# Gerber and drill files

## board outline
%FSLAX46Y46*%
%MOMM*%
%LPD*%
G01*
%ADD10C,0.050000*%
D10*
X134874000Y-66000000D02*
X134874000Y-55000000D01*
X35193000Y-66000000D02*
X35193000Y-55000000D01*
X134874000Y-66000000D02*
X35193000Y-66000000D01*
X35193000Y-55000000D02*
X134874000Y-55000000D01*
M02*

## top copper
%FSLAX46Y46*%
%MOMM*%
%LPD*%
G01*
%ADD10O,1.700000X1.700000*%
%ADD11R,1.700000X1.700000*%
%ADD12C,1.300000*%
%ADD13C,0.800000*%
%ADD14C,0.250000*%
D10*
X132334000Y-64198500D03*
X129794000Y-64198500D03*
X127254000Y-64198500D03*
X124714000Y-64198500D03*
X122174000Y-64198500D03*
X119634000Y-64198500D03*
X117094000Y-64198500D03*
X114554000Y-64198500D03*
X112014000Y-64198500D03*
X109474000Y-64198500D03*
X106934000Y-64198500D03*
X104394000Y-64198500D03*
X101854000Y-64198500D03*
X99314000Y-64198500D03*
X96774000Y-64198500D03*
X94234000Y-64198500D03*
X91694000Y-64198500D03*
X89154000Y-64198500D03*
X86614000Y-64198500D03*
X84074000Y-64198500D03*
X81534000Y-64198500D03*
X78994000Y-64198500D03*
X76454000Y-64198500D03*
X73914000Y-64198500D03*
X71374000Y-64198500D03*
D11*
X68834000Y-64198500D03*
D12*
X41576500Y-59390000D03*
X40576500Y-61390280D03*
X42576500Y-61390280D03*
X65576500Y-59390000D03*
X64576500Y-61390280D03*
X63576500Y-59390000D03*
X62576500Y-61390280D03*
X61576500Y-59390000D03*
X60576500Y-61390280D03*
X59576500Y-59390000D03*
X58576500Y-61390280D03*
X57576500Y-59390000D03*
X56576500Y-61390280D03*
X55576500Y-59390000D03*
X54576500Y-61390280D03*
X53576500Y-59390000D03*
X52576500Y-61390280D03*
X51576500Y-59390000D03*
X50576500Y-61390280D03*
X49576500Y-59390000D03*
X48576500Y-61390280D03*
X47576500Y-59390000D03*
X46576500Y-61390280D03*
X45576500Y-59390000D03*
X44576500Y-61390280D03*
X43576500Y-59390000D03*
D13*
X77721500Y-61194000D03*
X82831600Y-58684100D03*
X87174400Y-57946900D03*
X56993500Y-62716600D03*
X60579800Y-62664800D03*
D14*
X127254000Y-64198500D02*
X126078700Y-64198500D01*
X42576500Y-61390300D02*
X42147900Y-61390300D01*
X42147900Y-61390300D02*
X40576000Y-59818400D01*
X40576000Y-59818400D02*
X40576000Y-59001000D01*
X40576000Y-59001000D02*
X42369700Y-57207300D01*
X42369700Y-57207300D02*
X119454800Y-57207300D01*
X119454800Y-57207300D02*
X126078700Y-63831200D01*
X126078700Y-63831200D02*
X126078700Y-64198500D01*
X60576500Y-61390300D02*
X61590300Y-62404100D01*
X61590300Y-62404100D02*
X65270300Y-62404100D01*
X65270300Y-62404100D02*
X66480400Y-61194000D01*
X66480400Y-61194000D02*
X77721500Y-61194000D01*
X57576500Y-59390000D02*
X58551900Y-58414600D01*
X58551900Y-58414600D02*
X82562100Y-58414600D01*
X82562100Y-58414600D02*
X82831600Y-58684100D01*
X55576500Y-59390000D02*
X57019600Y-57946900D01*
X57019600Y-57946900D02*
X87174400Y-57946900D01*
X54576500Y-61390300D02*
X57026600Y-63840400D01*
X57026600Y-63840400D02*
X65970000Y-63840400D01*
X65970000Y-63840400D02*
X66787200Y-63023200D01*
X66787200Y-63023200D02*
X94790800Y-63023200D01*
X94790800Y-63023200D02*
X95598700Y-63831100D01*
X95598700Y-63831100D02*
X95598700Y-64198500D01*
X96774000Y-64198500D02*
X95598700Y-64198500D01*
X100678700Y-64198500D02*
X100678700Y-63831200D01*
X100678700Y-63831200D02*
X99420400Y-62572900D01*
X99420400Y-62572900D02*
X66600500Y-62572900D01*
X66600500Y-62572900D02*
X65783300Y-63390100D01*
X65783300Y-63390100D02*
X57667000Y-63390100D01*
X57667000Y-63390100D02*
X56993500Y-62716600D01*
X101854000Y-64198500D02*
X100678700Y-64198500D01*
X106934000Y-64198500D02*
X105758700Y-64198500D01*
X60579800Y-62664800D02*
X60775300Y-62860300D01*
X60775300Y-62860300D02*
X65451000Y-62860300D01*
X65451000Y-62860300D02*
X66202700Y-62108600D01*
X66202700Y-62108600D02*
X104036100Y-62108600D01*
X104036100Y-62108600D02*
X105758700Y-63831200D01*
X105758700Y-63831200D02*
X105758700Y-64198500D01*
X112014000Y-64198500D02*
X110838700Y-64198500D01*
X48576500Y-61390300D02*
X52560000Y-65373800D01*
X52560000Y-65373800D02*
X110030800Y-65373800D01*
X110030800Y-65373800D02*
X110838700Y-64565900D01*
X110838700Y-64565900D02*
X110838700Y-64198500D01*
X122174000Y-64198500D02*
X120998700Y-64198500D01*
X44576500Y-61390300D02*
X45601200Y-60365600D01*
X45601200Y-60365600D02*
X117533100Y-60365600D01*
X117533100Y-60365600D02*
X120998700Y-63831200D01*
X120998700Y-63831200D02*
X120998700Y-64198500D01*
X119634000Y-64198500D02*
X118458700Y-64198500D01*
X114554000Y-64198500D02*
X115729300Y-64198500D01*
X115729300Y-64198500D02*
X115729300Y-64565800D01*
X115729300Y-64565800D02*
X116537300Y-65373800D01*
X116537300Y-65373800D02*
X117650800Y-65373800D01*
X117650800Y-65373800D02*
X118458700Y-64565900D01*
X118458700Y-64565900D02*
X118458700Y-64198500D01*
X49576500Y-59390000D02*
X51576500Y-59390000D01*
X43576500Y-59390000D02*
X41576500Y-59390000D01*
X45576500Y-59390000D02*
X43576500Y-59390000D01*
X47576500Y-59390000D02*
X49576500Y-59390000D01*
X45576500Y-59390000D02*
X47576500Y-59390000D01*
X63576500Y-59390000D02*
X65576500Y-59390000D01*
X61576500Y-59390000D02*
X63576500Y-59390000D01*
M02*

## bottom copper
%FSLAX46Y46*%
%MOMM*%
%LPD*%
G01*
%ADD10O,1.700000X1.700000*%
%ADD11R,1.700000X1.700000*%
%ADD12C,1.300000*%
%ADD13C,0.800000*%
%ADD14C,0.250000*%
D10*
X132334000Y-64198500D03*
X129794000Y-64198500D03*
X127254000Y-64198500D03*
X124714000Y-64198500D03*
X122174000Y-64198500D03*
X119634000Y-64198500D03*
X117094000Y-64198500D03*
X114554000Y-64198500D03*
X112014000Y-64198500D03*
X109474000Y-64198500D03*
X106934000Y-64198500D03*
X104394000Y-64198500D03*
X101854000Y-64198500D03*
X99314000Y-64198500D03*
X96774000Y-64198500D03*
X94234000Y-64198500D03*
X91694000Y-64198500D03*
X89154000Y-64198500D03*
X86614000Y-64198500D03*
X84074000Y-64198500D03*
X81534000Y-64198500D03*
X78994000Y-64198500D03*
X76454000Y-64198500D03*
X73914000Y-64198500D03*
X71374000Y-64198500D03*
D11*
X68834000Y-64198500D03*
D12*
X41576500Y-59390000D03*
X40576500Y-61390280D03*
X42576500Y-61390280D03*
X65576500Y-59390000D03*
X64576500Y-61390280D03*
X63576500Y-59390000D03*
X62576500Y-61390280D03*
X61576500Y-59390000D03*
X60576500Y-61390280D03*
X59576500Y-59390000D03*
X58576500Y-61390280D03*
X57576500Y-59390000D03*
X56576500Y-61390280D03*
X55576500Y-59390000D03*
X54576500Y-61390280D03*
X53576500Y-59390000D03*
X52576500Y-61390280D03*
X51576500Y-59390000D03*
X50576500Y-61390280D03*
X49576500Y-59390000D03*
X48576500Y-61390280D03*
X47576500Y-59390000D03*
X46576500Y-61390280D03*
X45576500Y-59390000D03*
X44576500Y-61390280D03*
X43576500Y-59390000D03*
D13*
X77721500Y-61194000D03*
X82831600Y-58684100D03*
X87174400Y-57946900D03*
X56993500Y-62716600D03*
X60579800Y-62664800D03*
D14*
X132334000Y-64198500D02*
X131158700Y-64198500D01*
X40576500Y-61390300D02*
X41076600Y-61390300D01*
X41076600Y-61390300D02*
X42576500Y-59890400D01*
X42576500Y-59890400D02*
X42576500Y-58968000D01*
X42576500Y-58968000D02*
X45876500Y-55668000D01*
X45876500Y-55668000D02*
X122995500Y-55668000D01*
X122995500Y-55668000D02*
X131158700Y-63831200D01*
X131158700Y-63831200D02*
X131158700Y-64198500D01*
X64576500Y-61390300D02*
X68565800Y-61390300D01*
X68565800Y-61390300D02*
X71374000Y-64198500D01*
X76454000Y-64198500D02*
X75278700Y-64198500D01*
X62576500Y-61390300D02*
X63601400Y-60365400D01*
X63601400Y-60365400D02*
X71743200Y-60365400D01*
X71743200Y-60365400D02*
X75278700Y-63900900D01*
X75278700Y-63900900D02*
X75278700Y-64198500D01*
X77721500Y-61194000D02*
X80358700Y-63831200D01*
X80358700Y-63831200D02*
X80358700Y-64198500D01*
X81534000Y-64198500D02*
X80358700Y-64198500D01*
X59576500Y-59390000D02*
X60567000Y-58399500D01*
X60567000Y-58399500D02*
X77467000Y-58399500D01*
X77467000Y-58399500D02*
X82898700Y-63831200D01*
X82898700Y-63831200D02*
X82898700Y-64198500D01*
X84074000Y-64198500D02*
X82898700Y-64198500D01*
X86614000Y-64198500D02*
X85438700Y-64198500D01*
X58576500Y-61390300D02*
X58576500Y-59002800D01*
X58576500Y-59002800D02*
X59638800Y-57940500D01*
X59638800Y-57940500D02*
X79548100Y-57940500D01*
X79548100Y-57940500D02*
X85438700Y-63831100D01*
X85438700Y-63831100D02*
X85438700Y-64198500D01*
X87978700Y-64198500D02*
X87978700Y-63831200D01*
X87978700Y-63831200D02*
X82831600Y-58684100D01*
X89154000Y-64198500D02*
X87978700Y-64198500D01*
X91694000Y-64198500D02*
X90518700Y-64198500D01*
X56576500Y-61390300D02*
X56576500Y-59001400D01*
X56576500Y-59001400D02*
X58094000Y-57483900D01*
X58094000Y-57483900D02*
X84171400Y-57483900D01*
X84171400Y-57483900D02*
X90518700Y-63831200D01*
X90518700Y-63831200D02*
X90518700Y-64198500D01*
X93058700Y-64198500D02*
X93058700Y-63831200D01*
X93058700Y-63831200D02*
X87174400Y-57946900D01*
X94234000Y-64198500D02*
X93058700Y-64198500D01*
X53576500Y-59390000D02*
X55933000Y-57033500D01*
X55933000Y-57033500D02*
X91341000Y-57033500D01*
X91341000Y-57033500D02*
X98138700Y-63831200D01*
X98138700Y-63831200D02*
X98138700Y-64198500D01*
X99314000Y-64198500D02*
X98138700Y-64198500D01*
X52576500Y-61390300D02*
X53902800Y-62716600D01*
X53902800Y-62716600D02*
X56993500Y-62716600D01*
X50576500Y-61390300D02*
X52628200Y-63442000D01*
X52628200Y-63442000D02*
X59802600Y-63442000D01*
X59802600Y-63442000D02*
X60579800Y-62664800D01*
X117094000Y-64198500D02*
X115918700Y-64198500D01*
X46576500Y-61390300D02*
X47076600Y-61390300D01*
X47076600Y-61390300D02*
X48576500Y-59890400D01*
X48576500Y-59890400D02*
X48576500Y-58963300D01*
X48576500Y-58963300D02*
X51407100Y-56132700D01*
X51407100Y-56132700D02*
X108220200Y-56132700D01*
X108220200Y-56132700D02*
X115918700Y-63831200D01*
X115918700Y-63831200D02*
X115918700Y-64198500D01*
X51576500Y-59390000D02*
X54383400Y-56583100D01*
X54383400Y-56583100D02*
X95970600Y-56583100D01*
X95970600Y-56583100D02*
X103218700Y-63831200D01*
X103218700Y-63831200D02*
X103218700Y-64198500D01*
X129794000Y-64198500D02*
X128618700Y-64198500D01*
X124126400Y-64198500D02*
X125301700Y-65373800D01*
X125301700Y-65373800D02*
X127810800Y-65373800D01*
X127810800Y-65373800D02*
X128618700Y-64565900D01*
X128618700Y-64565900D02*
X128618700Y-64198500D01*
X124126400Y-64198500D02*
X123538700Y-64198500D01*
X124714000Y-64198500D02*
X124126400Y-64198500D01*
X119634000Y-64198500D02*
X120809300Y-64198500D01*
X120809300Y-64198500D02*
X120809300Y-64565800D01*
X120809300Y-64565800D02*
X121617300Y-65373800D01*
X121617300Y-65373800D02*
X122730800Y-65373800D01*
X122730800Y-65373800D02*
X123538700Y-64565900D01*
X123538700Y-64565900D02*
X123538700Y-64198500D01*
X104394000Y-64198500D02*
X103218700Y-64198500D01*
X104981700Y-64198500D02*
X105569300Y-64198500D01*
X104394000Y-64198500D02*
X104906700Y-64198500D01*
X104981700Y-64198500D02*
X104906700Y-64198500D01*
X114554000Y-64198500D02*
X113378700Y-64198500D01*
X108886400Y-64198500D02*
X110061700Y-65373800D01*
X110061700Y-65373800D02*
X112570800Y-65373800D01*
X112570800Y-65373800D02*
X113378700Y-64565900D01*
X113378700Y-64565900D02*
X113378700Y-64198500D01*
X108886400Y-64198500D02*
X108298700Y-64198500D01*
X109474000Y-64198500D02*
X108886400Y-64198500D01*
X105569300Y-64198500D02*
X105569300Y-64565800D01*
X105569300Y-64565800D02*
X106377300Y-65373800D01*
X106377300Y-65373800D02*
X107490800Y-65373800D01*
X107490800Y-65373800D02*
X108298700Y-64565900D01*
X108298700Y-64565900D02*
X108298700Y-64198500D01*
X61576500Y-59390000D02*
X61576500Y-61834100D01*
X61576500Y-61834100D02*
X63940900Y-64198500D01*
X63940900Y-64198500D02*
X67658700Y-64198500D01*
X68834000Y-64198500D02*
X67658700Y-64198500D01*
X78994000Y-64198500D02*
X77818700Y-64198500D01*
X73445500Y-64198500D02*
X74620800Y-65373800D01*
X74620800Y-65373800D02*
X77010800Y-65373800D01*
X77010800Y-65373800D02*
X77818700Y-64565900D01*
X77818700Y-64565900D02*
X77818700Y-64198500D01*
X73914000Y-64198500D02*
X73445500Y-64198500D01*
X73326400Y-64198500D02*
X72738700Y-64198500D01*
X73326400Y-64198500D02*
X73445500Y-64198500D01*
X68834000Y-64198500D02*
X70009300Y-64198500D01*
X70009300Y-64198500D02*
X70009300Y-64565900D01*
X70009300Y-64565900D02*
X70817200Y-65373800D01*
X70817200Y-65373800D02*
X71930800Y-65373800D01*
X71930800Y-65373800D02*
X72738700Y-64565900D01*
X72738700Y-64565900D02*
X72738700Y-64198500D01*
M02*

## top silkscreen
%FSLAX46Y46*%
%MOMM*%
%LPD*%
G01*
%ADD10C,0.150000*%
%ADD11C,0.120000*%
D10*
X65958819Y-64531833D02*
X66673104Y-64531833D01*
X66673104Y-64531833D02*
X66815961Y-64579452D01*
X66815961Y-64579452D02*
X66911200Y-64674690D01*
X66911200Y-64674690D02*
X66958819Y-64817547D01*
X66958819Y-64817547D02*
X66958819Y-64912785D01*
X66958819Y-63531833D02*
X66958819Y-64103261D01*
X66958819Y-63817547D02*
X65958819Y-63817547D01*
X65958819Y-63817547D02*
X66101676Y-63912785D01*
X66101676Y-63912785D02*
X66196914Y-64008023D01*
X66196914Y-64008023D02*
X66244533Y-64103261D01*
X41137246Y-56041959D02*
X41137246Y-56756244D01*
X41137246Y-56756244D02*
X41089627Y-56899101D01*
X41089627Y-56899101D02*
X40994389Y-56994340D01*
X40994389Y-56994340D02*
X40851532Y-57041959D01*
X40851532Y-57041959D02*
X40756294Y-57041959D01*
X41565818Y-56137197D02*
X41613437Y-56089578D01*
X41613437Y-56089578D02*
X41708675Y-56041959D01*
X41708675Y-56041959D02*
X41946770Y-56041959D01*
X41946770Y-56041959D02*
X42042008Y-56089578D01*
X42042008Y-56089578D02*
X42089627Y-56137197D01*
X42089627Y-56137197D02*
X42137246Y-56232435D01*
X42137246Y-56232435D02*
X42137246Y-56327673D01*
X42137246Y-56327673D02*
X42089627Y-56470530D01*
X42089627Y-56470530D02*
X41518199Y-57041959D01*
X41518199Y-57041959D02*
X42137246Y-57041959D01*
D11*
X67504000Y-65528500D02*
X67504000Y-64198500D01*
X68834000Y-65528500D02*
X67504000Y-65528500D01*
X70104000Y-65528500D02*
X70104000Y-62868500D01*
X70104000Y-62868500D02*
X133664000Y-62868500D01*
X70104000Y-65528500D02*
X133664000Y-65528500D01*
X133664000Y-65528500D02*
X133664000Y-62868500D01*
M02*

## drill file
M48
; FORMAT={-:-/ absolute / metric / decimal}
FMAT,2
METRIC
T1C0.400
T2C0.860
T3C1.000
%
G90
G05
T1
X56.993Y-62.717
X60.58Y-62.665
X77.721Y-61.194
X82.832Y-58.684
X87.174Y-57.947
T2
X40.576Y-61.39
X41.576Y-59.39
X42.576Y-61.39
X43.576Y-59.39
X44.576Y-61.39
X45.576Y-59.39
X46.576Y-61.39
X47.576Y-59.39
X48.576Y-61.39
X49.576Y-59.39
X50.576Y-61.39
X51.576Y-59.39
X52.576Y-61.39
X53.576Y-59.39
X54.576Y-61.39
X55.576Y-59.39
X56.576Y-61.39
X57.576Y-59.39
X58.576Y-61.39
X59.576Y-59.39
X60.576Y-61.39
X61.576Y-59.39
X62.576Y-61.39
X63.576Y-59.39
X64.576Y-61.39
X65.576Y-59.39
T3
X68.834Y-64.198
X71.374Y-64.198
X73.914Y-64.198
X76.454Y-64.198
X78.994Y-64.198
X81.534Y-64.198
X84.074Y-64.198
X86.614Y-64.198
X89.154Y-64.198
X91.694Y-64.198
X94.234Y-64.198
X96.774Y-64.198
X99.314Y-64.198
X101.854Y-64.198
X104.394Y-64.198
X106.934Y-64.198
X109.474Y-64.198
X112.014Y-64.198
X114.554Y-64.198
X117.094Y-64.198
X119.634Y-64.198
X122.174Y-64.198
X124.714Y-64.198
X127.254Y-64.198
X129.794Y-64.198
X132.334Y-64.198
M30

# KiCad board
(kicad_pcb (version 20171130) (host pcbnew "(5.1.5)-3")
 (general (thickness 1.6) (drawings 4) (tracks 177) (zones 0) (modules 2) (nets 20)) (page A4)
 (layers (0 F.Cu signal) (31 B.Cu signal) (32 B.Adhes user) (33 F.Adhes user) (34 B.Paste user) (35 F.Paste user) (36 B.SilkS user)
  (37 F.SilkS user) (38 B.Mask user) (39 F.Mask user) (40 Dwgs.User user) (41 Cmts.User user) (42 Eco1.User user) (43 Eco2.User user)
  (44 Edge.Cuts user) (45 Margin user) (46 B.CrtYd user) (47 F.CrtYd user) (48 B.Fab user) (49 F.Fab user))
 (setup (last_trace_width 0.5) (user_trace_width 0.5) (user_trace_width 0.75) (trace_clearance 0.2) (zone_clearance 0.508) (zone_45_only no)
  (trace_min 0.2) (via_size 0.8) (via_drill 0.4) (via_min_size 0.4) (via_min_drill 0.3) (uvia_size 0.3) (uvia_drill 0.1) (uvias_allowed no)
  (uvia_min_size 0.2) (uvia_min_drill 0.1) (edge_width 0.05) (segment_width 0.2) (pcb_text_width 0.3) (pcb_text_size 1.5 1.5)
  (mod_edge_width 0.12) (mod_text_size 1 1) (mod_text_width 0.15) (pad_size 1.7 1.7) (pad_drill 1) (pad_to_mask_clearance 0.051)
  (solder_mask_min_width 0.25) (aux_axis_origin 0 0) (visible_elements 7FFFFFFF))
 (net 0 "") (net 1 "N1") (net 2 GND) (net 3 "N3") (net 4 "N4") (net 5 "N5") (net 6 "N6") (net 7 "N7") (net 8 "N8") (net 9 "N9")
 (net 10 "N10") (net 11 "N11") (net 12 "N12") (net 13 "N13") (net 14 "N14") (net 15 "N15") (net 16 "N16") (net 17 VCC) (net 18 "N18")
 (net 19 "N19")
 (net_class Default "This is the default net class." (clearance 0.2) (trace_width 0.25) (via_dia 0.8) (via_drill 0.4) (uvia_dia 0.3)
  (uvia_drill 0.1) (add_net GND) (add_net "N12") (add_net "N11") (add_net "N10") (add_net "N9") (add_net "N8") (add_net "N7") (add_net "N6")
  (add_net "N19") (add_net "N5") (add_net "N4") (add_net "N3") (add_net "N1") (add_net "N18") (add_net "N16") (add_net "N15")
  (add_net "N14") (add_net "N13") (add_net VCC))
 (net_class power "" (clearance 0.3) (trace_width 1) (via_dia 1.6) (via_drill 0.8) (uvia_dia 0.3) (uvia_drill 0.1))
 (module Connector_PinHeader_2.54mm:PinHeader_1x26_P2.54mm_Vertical (layer F.Cu) (at 68.834 64.1985 90)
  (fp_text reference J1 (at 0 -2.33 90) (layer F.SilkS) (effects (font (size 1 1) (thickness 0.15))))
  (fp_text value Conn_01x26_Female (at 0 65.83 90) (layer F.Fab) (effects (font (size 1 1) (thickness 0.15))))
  (fp_line (start -1.33 -1.33) (end 0 -1.33) (layer F.SilkS) (width 0.12))
  (fp_line (start -1.33 0) (end -1.33 -1.33) (layer F.SilkS) (width 0.12))
  (fp_line (start -1.33 1.27) (end 1.33 1.27) (layer F.SilkS) (width 0.12))
  (fp_line (start 1.33 1.27) (end 1.33 64.83) (layer F.SilkS) (width 0.12))
  (fp_line (start -1.33 1.27) (end -1.33 64.83) (layer F.SilkS) (width 0.12))
  (fp_line (start -1.33 64.83) (end 1.33 64.83) (layer F.SilkS) (width 0.12))
  (pad 26 thru_hole oval (at 0 63.5 90) (size 1.7 1.7) (drill 1) (layers *.Cu *.Mask) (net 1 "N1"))
  (pad 25 thru_hole oval (at 0 60.96 90) (size 1.7 1.7) (drill 1) (layers *.Cu *.Mask) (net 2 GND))
  (pad 24 thru_hole oval (at 0 58.42 90) (size 1.7 1.7) (drill 1) (layers *.Cu *.Mask) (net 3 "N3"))
  (pad 23 thru_hole oval (at 0 55.88 90) (size 1.7 1.7) (drill 1) (layers *.Cu *.Mask) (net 2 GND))
  (pad 22 thru_hole oval (at 0 53.34 90) (size 1.7 1.7) (drill 1) (layers *.Cu *.Mask) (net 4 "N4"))
  (pad 21 thru_hole oval (at 0 50.8 90) (size 1.7 1.7) (drill 1) (layers *.Cu *.Mask) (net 2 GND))
  (pad 20 thru_hole oval (at 0 48.26 90) (size 1.7 1.7) (drill 1) (layers *.Cu *.Mask) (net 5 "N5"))
  (pad 19 thru_hole oval (at 0 45.72 90) (size 1.7 1.7) (drill 1) (layers *.Cu *.Mask) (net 2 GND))
  (pad 18 thru_hole oval (at 0 43.18 90) (size 1.7 1.7) (drill 1) (layers *.Cu *.Mask) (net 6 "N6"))
  (pad 17 thru_hole oval (at 0 40.64 90) (size 1.7 1.7) (drill 1) (layers *.Cu *.Mask) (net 2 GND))
  (pad 16 thru_hole oval (at 0 38.1 90) (size 1.7 1.7) (drill 1) (layers *.Cu *.Mask) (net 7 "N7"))
  (pad 15 thru_hole oval (at 0 35.56 90) (size 1.7 1.7) (drill 1) (layers *.Cu *.Mask) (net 2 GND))
  (pad 14 thru_hole oval (at 0 33.02 90) (size 1.7 1.7) (drill 1) (layers *.Cu *.Mask) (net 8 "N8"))
  (pad 13 thru_hole oval (at 0 30.48 90) (size 1.7 1.7) (drill 1) (layers *.Cu *.Mask) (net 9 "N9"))
  (pad 12 thru_hole oval (at 0 27.94 90) (size 1.7 1.7) (drill 1) (layers *.Cu *.Mask) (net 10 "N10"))
  (pad 11 thru_hole oval (at 0 25.4 90) (size 1.7 1.7) (drill 1) (layers *.Cu *.Mask) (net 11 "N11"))
  (pad 10 thru_hole oval (at 0 22.86 90) (size 1.7 1.7) (drill 1) (layers *.Cu *.Mask) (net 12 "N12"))
  (pad 9 thru_hole oval (at 0 20.32 90) (size 1.7 1.7) (drill 1) (layers *.Cu *.Mask) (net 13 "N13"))
  (pad 8 thru_hole oval (at 0 17.78 90) (size 1.7 1.7) (drill 1) (layers *.Cu *.Mask) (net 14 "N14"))
  (pad 7 thru_hole oval (at 0 15.24 90) (size 1.7 1.7) (drill 1) (layers *.Cu *.Mask) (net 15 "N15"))
  (pad 6 thru_hole oval (at 0 12.7 90) (size 1.7 1.7) (drill 1) (layers *.Cu *.Mask) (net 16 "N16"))
  (pad 5 thru_hole oval (at 0 10.16 90) (size 1.7 1.7) (drill 1) (layers *.Cu *.Mask) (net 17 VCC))
  (pad 4 thru_hole oval (at 0 7.62 90) (size 1.7 1.7) (drill 1) (layers *.Cu *.Mask) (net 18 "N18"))
  (pad 3 thru_hole oval (at 0 5.08 90) (size 1.7 1.7) (drill 1) (layers *.Cu *.Mask) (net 17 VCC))
  (pad 2 thru_hole oval (at 0 2.54 90) (size 1.7 1.7) (drill 1) (layers *.Cu *.Mask) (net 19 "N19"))
  (pad 1 thru_hole rect (at 0 0 90) (size 1.7 1.7) (drill 1) (layers *.Cu *.Mask) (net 17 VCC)))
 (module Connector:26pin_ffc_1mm (layer F.Cu) (at 40.5765 64.103)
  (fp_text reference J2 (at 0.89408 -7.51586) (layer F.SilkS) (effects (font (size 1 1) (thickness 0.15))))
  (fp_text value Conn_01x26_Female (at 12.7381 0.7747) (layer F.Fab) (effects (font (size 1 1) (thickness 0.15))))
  (pad 25 thru_hole circle (at 1 -4.713) (size 1.3 1.3) (drill 0.86) (layers *.Cu *.Mask) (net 2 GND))
  (pad 26 thru_hole circle (at 0 -2.71272) (size 1.3 1.3) (drill 0.86) (layers *.Cu *.Mask) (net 1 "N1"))
  (pad 24 thru_hole circle (at 2 -2.71272) (size 1.3 1.3) (drill 0.86) (layers *.Cu *.Mask) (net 3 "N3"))
  (pad 1 thru_hole circle (at 25 -4.713) (size 1.3 1.3) (drill 0.86) (layers *.Cu *.Mask) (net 17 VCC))
  (pad 2 thru_hole circle (at 24 -2.71272) (size 1.3 1.3) (drill 0.86) (layers *.Cu *.Mask) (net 19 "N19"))
  (pad 3 thru_hole circle (at 23 -4.713) (size 1.3 1.3) (drill 0.86) (layers *.Cu *.Mask) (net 17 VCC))
  (pad 4 thru_hole circle (at 22 -2.71272) (size 1.3 1.3) (drill 0.86) (layers *.Cu *.Mask) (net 18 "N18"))
  (pad 5 thru_hole circle (at 21 -4.713) (size 1.3 1.3) (drill 0.86) (layers *.Cu *.Mask) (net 17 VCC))
  (pad 6 thru_hole circle (at 20 -2.71272) (size 1.3 1.3) (drill 0.86) (layers *.Cu *.Mask) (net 16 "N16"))
  (pad 7 thru_hole circle (at 19 -4.713) (size 1.3 1.3) (drill 0.86) (layers *.Cu *.Mask) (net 15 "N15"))
  (pad 8 thru_hole circle (at 18 -2.71272) (size 1.3 1.3) (drill 0.86) (layers *.Cu *.Mask) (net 14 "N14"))
  (pad 9 thru_hole circle (at 17 -4.713) (size 1.3 1.3) (drill 0.86) (layers *.Cu *.Mask) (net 13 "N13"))
  (pad 10 thru_hole circle (at 16 -2.71272) (size 1.3 1.3) (drill 0.86) (layers *.Cu *.Mask) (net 12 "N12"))
  (pad 11 thru_hole circle (at 15 -4.713) (size 1.3 1.3) (drill 0.86) (layers *.Cu *.Mask) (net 11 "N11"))
  (pad 12 thru_hole circle (at 14 -2.71272) (size 1.3 1.3) (drill 0.86) (layers *.Cu *.Mask) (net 10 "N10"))
  (pad 13 thru_hole circle (at 13 -4.713) (size 1.3 1.3) (drill 0.86) (layers *.Cu *.Mask) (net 9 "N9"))
  (pad 14 thru_hole circle (at 12 -2.71272) (size 1.3 1.3) (drill 0.86) (layers *.Cu *.Mask) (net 8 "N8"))
  (pad 15 thru_hole circle (at 11 -4.713) (size 1.3 1.3) (drill 0.86) (layers *.Cu *.Mask) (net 2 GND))
  (pad 16 thru_hole circle (at 10 -2.71272) (size 1.3 1.3) (drill 0.86) (layers *.Cu *.Mask) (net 7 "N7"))
  (pad 17 thru_hole circle (at 9 -4.713) (size 1.3 1.3) (drill 0.86) (layers *.Cu *.Mask) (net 2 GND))
  (pad 18 thru_hole circle (at 8 -2.71272) (size 1.3 1.3) (drill 0.86) (layers *.Cu *.Mask) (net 6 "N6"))
  (pad 19 thru_hole circle (at 7 -4.713) (size 1.3 1.3) (drill 0.86) (layers *.Cu *.Mask) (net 2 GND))
  (pad 20 thru_hole circle (at 6 -2.71272) (size 1.3 1.3) (drill 0.86) (layers *.Cu *.Mask) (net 5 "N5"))
  (pad 21 thru_hole circle (at 5 -4.713) (size 1.3 1.3) (drill 0.86) (layers *.Cu *.Mask) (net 2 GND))
  (pad 22 thru_hole circle (at 4 -2.71272) (size 1.3 1.3) (drill 0.86) (layers *.Cu *.Mask) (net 4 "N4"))
  (pad 23 thru_hole circle (at 3 -4.713) (size 1.3 1.3) (drill 0.86) (layers *.Cu *.Mask) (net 2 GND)))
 (gr_line (start 134.874 66) (end 134.874 55) (layer Edge.Cuts) (width 0.05))
 (gr_line (start 35.193 66) (end 35.193 55) (layer Edge.Cuts) (width 0.05))
 (gr_line (start 134.874 66) (end 35.193 66) (layer Edge.Cuts) (width 0.05))
 (gr_line (start 35.193 55) (end 134.874 55) (layer Edge.Cuts) (width 0.05))
 (segment (start 132.334 64.1985) (end 131.1587 64.1985) (width 0.25) (layer B.Cu) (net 1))
 (segment (start 40.5765 61.3903) (end 41.0766 61.3903) (width 0.25) (layer B.Cu) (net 1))
 (segment (start 41.0766 61.3903) (end 42.5765 59.8904) (width 0.25) (layer B.Cu) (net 1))
 (segment (start 42.5765 59.8904) (end 42.5765 58.968) (width 0.25) (layer B.Cu) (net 1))
 (segment (start 42.5765 58.968) (end 45.8765 55.668) (width 0.25) (layer B.Cu) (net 1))
 (segment (start 45.8765 55.668) (end 122.9955 55.668) (width 0.25) (layer B.Cu) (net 1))
 (segment (start 122.9955 55.668) (end 131.1587 63.8312) (width 0.25) (layer B.Cu) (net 1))
 (segment (start 131.1587 63.8312) (end 131.1587 64.1985) (width 0.25) (layer B.Cu) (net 1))
 (segment (start 127.254 64.1985) (end 126.0787 64.1985) (width 0.25) (layer F.Cu) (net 3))
 (segment (start 42.5765 61.3903) (end 42.1479 61.3903) (width 0.25) (layer F.Cu) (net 3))
 (segment (start 42.1479 61.3903) (end 40.576 59.8184) (width 0.25) (layer F.Cu) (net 3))
 (segment (start 40.576 59.8184) (end 40.576 59.001) (width 0.25) (layer F.Cu) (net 3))
 (segment (start 40.576 59.001) (end 42.3697 57.2073) (width 0.25) (layer F.Cu) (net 3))
 (segment (start 42.3697 57.2073) (end 119.4548 57.2073) (width 0.25) (layer F.Cu) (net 3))
 (segment (start 119.4548 57.2073) (end 126.0787 63.8312) (width 0.25) (layer F.Cu) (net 3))
 (segment (start 126.0787 63.8312) (end 126.0787 64.1985) (width 0.25) (layer F.Cu) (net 3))
 (segment (start 64.5765 61.3903) (end 68.5658 61.3903) (width 0.25) (layer B.Cu) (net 19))
 (segment (start 68.5658 61.3903) (end 71.374 64.1985) (width 0.25) (layer B.Cu) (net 19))
 (segment (start 76.454 64.1985) (end 75.2787 64.1985) (width 0.25) (layer B.Cu) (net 18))
 (segment (start 62.5765 61.3903) (end 63.6014 60.3654) (width 0.25) (layer B.Cu) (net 18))
 (segment (start 63.6014 60.3654) (end 71.7432 60.3654) (width 0.25) (layer B.Cu) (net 18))
 (segment (start 71.7432 60.3654) (end 75.2787 63.9009) (width 0.25) (layer B.Cu) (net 18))
 (segment (start 75.2787 63.9009) (end 75.2787 64.1985) (width 0.25) (layer B.Cu) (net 18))
 (segment (start 60.5765 61.3903) (end 61.5903 62.4041) (width 0.25) (layer F.Cu) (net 16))
 (segment (start 61.5903 62.4041) (end 65.2703 62.4041) (width 0.25) (layer F.Cu) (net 16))
 (segment (start 65.2703 62.4041) (end 66.4804 61.194) (width 0.25) (layer F.Cu) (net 16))
 (segment (start 66.4804 61.194) (end 77.7215 61.194) (width 0.25) (layer F.Cu) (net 16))
 (segment (start 77.7215 61.194) (end 80.3587 63.8312) (width 0.25) (layer B.Cu) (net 16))
 (segment (start 80.3587 63.8312) (end 80.3587 64.1985) (width 0.25) (layer B.Cu) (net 16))
 (segment (start 81.534 64.1985) (end 80.3587 64.1985) (width 0.25) (layer B.Cu) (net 16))
 (via (at 77.7215 61.194) (size 0.8) (layers F.Cu B.Cu) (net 16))
 (segment (start 59.5765 59.39) (end 60.567 58.3995) (width 0.25) (layer B.Cu) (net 15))
 (segment (start 60.567 58.3995) (end 77.467 58.3995) (width 0.25) (layer B.Cu) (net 15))
 (segment (start 77.467 58.3995) (end 82.8987 63.8312) (width 0.25) (layer B.Cu) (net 15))
 (segment (start 82.8987 63.8312) (end 82.8987 64.1985) (width 0.25) (layer B.Cu) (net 15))
 (segment (start 84.074 64.1985) (end 82.8987 64.1985) (width 0.25) (layer B.Cu) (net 15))
 (segment (start 86.614 64.1985) (end 85.4387 64.1985) (width 0.25) (layer B.Cu) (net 14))
 (segment (start 58.5765 61.3903) (end 58.5765 59.0028) (width 0.25) (layer B.Cu) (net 14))
 (segment (start 58.5765 59.0028) (end 59.6388 57.9405) (width 0.25) (layer B.Cu) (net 14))
 (segment (start 59.6388 57.9405) (end 79.5481 57.9405) (width 0.25) (layer B.Cu) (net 14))
 (segment (start 79.5481 57.9405) (end 85.4387 63.8311) (width 0.25) (layer B.Cu) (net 14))
 (segment (start 85.4387 63.8311) (end 85.4387 64.1985) (width 0.25) (layer B.Cu) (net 14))
 (segment (start 57.5765 59.39) (end 58.5519 58.4146) (width 0.25) (layer F.Cu) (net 13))
 (segment (start 58.5519 58.4146) (end 82.5621 58.4146) (width 0.25) (layer F.Cu) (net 13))
 (segment (start 82.5621 58.4146) (end 82.8316 58.6841) (width 0.25) (layer F.Cu) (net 13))
 (segment (start 87.9787 64.1985) (end 87.9787 63.8312) (width 0.25) (layer B.Cu) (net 13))
 (segment (start 87.9787 63.8312) (end 82.8316 58.6841) (width 0.25) (layer B.Cu) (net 13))
 (segment (start 89.154 64.1985) (end 87.9787 64.1985) (width 0.25) (layer B.Cu) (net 13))
 (via (at 82.8316 58.6841) (size 0.8) (layers F.Cu B.Cu) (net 13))
 (segment (start 91.694 64.1985) (end 90.5187 64.1985) (width 0.25) (layer B.Cu) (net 12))
 (segment (start 56.5765 61.3903) (end 56.5765 59.0014) (width 0.25) (layer B.Cu) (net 12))
 (segment (start 56.5765 59.0014) (end 58.094 57.4839) (width 0.25) (layer B.Cu) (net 12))
 (segment (start 58.094 57.4839) (end 84.1714 57.4839) (width 0.25) (layer B.Cu) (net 12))
 (segment (start 84.1714 57.4839) (end 90.5187 63.8312) (width 0.25) (layer B.Cu) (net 12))
 (segment (start 90.5187 63.8312) (end 90.5187 64.1985) (width 0.25) (layer B.Cu) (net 12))
 (segment (start 55.5765 59.39) (end 57.0196 57.9469) (width 0.25) (layer F.Cu) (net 11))
 (segment (start 57.0196 57.9469) (end 87.1744 57.9469) (width 0.25) (layer F.Cu) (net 11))
 (segment (start 93.0587 64.1985) (end 93.0587 63.8312) (width 0.25) (layer B.Cu) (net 11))
 (segment (start 93.0587 63.8312) (end 87.1744 57.9469) (width 0.25) (layer B.Cu) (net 11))
 (segment (start 94.234 64.1985) (end 93.0587 64.1985) (width 0.25) (layer B.Cu) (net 11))
 (via (at 87.1744 57.9469) (size 0.8) (layers F.Cu B.Cu) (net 11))
 (segment (start 54.5765 61.3903) (end 57.0266 63.8404) (width 0.25) (layer F.Cu) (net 10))
 (segment (start 57.0266 63.8404) (end 65.97 63.8404) (width 0.25) (layer F.Cu) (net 10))
 (segment (start 65.97 63.8404) (end 66.7872 63.0232) (width 0.25) (layer F.Cu) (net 10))
 (segment (start 66.7872 63.0232) (end 94.7908 63.0232) (width 0.25) (layer F.Cu) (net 10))
 (segment (start 94.7908 63.0232) (end 95.5987 63.8311) (width 0.25) (layer F.Cu) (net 10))
 (segment (start 95.5987 63.8311) (end 95.5987 64.1985) (width 0.25) (layer F.Cu) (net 10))
 (segment (start 96.774 64.1985) (end 95.5987 64.1985) (width 0.25) (layer F.Cu) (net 10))
 (segment (start 53.5765 59.39) (end 55.933 57.0335) (width 0.25) (layer B.Cu) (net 9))
 (segment (start 55.933 57.0335) (end 91.341 57.0335) (width 0.25) (layer B.Cu) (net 9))
 (segment (start 91.341 57.0335) (end 98.1387 63.8312) (width 0.25) (layer B.Cu) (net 9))
 (segment (start 98.1387 63.8312) (end 98.1387 64.1985) (width 0.25) (layer B.Cu) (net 9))
 (segment (start 99.314 64.1985) (end 98.1387 64.1985) (width 0.25) (layer B.Cu) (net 9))
 (segment (start 100.6787 64.1985) (end 100.6787 63.8312) (width 0.25) (layer F.Cu) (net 8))
 (segment (start 100.6787 63.8312) (end 99.4204 62.5729) (width 0.25) (layer F.Cu) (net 8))
 (segment (start 99.4204 62.5729) (end 66.6005 62.5729) (width 0.25) (layer F.Cu) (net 8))
 (segment (start 66.6005 62.5729) (end 65.7833 63.3901) (width 0.25) (layer F.Cu) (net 8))
 (segment (start 65.7833 63.3901) (end 57.667 63.3901) (width 0.25) (layer F.Cu) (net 8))
 (segment (start 57.667 63.3901) (end 56.9935 62.7166) (width 0.25) (layer F.Cu) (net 8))
 (segment (start 52.5765 61.3903) (end 53.9028 62.7166) (width 0.25) (layer B.Cu) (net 8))
 (segment (start 53.9028 62.7166) (end 56.9935 62.7166) (width 0.25) (layer B.Cu) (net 8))
 (segment (start 101.854 64.1985) (end 100.6787 64.1985) (width 0.25) (layer F.Cu) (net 8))
 (via (at 56.9935 62.7166) (size 0.8) (layers F.Cu B.Cu) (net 8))
 (segment (start 106.934 64.1985) (end 105.7587 64.1985) (width 0.25) (layer F.Cu) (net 7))
 (segment (start 60.5798 62.6648) (end 60.7753 62.8603) (width 0.25) (layer F.Cu) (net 7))
 (segment (start 60.7753 62.8603) (end 65.451 62.8603) (width 0.25) (layer F.Cu) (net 7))
 (segment (start 65.451 62.8603) (end 66.2027 62.1086) (width 0.25) (layer F.Cu) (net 7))
 (segment (start 66.2027 62.1086) (end 104.0361 62.1086) (width 0.25) (layer F.Cu) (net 7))
 (segment (start 104.0361 62.1086) (end 105.7587 63.8312) (width 0.25) (layer F.Cu) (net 7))
 (segment (start 105.7587 63.8312) (end 105.7587 64.1985) (width 0.25) (layer F.Cu) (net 7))
 (segment (start 50.5765 61.3903) (end 52.6282 63.442) (width 0.25) (layer B.Cu) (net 7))
 (segment (start 52.6282 63.442) (end 59.8026 63.442) (width 0.25) (layer B.Cu) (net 7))
 (segment (start 59.8026 63.442) (end 60.5798 62.6648) (width 0.25) (layer B.Cu) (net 7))
 (via (at 60.5798 62.6648) (size 0.8) (layers F.Cu B.Cu) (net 7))
 (segment (start 112.014 64.1985) (end 110.8387 64.1985) (width 0.25) (layer F.Cu) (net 6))
 (segment (start 48.5765 61.3903) (end 52.56 65.3738) (width 0.25) (layer F.Cu) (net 6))
 (segment (start 52.56 65.3738) (end 110.0308 65.3738) (width 0.25) (layer F.Cu) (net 6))
 (segment (start 110.0308 65.3738) (end 110.8387 64.5659) (width 0.25) (layer F.Cu) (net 6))
 (segment (start 110.8387 64.5659) (end 110.8387 64.1985) (width 0.25) (layer F.Cu) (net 6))
 (segment (start 117.094 64.1985) (end 115.9187 64.1985) (width 0.25) (layer B.Cu) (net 5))
 (segment (start 46.5765 61.3903) (end 47.0766 61.3903) (width 0.25) (layer B.Cu) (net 5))
 (segment (start 47.0766 61.3903) (end 48.5765 59.8904) (width 0.25) (layer B.Cu) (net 5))
 (segment (start 48.5765 59.8904) (end 48.5765 58.9633) (width 0.25) (layer B.Cu) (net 5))
 (segment (start 48.5765 58.9633) (end 51.4071 56.1327) (width 0.25) (layer B.Cu) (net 5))
 (segment (start 51.4071 56.1327) (end 108.2202 56.1327) (width 0.25) (layer B.Cu) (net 5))
 (segment (start 108.2202 56.1327) (end 115.9187 63.8312) (width 0.25) (layer B.Cu) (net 5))
 (segment (start 115.9187 63.8312) (end 115.9187 64.1985) (width 0.25) (layer B.Cu) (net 5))
 (segment (start 122.174 64.1985) (end 120.9987 64.1985) (width 0.25) (layer F.Cu) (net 4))
 (segment (start 44.5765 61.3903) (end 45.6012 60.3656) (width 0.25) (layer F.Cu) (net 4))
 (segment (start 45.6012 60.3656) (end 117.5331 60.3656) (width 0.25) (layer F.Cu) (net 4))
 (segment (start 117.5331 60.3656) (end 120.9987 63.8312) (width 0.25) (layer F.Cu) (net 4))
 (segment (start 120.9987 63.8312) (end 120.9987 64.1985) (width 0.25) (layer F.Cu) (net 4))
 (segment (start 51.5765 59.39) (end 54.3834 56.5831) (width 0.25) (layer B.Cu) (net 2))
 (segment (start 54.3834 56.5831) (end 95.9706 56.5831) (width 0.25) (layer B.Cu) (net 2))
 (segment (start 95.9706 56.5831) (end 103.2187 63.8312) (width 0.25) (layer B.Cu) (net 2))
 (segment (start 103.2187 63.8312) (end 103.2187 64.1985) (width 0.25) (layer B.Cu) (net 2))
 (segment (start 129.794 64.1985) (end 128.6187 64.1985) (width 0.25) (layer B.Cu) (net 2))
 (segment (start 124.1264 64.1985) (end 125.3017 65.3738) (width 0.25) (layer B.Cu) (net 2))
 (segment (start 125.3017 65.3738) (end 127.8108 65.3738) (width 0.25) (layer B.Cu) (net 2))
 (segment (start 127.8108 65.3738) (end 128.6187 64.5659) (width 0.25) (layer B.Cu) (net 2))
 (segment (start 128.6187 64.5659) (end 128.6187 64.1985) (width 0.25) (layer B.Cu) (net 2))
 (segment (start 124.1264 64.1985) (end 123.5387 64.1985) (width 0.25) (layer B.Cu) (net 2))
 (segment (start 124.714 64.1985) (end 124.1264 64.1985) (width 0.25) (layer B.Cu) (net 2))
 (segment (start 119.634 64.1985) (end 120.8093 64.1985) (width 0.25) (layer B.Cu) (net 2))
 (segment (start 120.8093 64.1985) (end 120.8093 64.5658) (width 0.25) (layer B.Cu) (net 2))
 (segment (start 120.8093 64.5658) (end 121.6173 65.3738) (width 0.25) (layer B.Cu) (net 2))
 (segment (start 121.6173 65.3738) (end 122.7308 65.3738) (width 0.25) (layer B.Cu) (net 2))
 (segment (start 122.7308 65.3738) (end 123.5387 64.5659) (width 0.25) (layer B.Cu) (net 2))
 (segment (start 123.5387 64.5659) (end 123.5387 64.1985) (width 0.25) (layer B.Cu) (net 2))
 (segment (start 119.634 64.1985) (end 118.4587 64.1985) (width 0.25) (layer F.Cu) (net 2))
 (segment (start 114.554 64.1985) (end 115.7293 64.1985) (width 0.25) (layer F.Cu) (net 2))
 (segment (start 115.7293 64.1985) (end 115.7293 64.5658) (width 0.25) (layer F.Cu) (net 2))
 (segment (start 115.7293 64.5658) (end 116.5373 65.3738) (width 0.25) (layer F.Cu) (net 2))
 (segment (start 116.5373 65.3738) (end 117.6508 65.3738) (width 0.25) (layer F.Cu) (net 2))
 (segment (start 117.6508 65.3738) (end 118.4587 64.5659) (width 0.25) (layer F.Cu) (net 2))
 (segment (start 118.4587 64.5659) (end 118.4587 64.1985) (width 0.25) (layer F.Cu) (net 2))
 (segment (start 104.394 64.1985) (end 103.2187 64.1985) (width 0.25) (layer B.Cu) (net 2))
 (segment (start 49.5765 59.39) (end 51.5765 59.39) (width 0.25) (layer F.Cu) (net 2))
 (segment (start 104.9817 64.1985) (end 105.5693 64.1985) (width 0.25) (layer B.Cu) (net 2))
 (segment (start 104.394 64.1985) (end 104.9067 64.1985) (width 0.25) (layer B.Cu) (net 2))
 (segment (start 104.9817 64.1985) (end 104.9067 64.1985) (width 0.25) (layer B.Cu) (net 2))
 (segment (start 114.554 64.1985) (end 113.3787 64.1985) (width 0.25) (layer B.Cu) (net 2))
 (segment (start 108.8864 64.1985) (end 110.0617 65.3738) (width 0.25) (layer B.Cu) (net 2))
 (segment (start 110.0617 65.3738) (end 112.5708 65.3738) (width 0.25) (layer B.Cu) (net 2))
 (segment (start 112.5708 65.3738) (end 113.3787 64.5659) (width 0.25) (layer B.Cu) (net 2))
 (segment (start 113.3787 64.5659) (end 113.3787 64.1985) (width 0.25) (layer B.Cu) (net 2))
 (segment (start 108.8864 64.1985) (end 108.2987 64.1985) (width 0.25) (layer B.Cu) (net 2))
 (segment (start 109.474 64.1985) (end 108.8864 64.1985) (width 0.25) (layer B.Cu) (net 2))
 (segment (start 105.5693 64.1985) (end 105.5693 64.5658) (width 0.25) (layer B.Cu) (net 2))
 (segment (start 105.5693 64.5658) (end 106.3773 65.3738) (width 0.25) (layer B.Cu) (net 2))
 (segment (start 106.3773 65.3738) (end 107.4908 65.3738) (width 0.25) (layer B.Cu) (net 2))
 (segment (start 107.4908 65.3738) (end 108.2987 64.5659) (width 0.25) (layer B.Cu) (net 2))
 (segment (start 108.2987 64.5659) (end 108.2987 64.1985) (width 0.25) (layer B.Cu) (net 2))
 (segment (start 43.5765 59.39) (end 41.5765 59.39) (width 0.25) (layer F.Cu) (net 2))
 (segment (start 45.5765 59.39) (end 43.5765 59.39) (width 0.25) (layer F.Cu) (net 2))
 (segment (start 47.5765 59.39) (end 49.5765 59.39) (width 0.25) (layer F.Cu) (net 2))
 (segment (start 45.5765 59.39) (end 47.5765 59.39) (width 0.25) (layer F.Cu) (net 2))
 (segment (start 61.5765 59.39) (end 61.5765 61.8341) (width 0.25) (layer B.Cu) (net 17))
 (segment (start 61.5765 61.8341) (end 63.9409 64.1985) (width 0.25) (layer B.Cu) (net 17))
 (segment (start 63.9409 64.1985) (end 67.6587 64.1985) (width 0.25) (layer B.Cu) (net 17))
 (segment (start 68.834 64.1985) (end 67.6587 64.1985) (width 0.25) (layer B.Cu) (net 17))
 (segment (start 78.994 64.1985) (end 77.8187 64.1985) (width 0.25) (layer B.Cu) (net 17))
 (segment (start 73.4455 64.1985) (end 74.6208 65.3738) (width 0.25) (layer B.Cu) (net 17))
 (segment (start 74.6208 65.3738) (end 77.0108 65.3738) (width 0.25) (layer B.Cu) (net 17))
 (segment (start 77.0108 65.3738) (end 77.8187 64.5659) (width 0.25) (layer B.Cu) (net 17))
 (segment (start 77.8187 64.5659) (end 77.8187 64.1985) (width 0.25) (layer B.Cu) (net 17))
 (segment (start 73.914 64.1985) (end 73.4455 64.1985) (width 0.25) (layer B.Cu) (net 17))
 (segment (start 73.3264 64.1985) (end 72.7387 64.1985) (width 0.25) (layer B.Cu) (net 17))
 (segment (start 73.3264 64.1985) (end 73.4455 64.1985) (width 0.25) (layer B.Cu) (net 17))
 (segment (start 68.834 64.1985) (end 70.0093 64.1985) (width 0.25) (layer B.Cu) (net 17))
 (segment (start 70.0093 64.1985) (end 70.0093 64.5659) (width 0.25) (layer B.Cu) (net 17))
 (segment (start 70.0093 64.5659) (end 70.8172 65.3738) (width 0.25) (layer B.Cu) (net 17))
 (segment (start 70.8172 65.3738) (end 71.9308 65.3738) (width 0.25) (layer B.Cu) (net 17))
 (segment (start 71.9308 65.3738) (end 72.7387 64.5659) (width 0.25) (layer B.Cu) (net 17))
 (segment (start 72.7387 64.5659) (end 72.7387 64.1985) (width 0.25) (layer B.Cu) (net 17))
 (segment (start 63.5765 59.39) (end 65.5765 59.39) (width 0.25) (layer F.Cu) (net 17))
 (segment (start 61.5765 59.39) (end 63.5765 59.39) (width 0.25) (layer F.Cu) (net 17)))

